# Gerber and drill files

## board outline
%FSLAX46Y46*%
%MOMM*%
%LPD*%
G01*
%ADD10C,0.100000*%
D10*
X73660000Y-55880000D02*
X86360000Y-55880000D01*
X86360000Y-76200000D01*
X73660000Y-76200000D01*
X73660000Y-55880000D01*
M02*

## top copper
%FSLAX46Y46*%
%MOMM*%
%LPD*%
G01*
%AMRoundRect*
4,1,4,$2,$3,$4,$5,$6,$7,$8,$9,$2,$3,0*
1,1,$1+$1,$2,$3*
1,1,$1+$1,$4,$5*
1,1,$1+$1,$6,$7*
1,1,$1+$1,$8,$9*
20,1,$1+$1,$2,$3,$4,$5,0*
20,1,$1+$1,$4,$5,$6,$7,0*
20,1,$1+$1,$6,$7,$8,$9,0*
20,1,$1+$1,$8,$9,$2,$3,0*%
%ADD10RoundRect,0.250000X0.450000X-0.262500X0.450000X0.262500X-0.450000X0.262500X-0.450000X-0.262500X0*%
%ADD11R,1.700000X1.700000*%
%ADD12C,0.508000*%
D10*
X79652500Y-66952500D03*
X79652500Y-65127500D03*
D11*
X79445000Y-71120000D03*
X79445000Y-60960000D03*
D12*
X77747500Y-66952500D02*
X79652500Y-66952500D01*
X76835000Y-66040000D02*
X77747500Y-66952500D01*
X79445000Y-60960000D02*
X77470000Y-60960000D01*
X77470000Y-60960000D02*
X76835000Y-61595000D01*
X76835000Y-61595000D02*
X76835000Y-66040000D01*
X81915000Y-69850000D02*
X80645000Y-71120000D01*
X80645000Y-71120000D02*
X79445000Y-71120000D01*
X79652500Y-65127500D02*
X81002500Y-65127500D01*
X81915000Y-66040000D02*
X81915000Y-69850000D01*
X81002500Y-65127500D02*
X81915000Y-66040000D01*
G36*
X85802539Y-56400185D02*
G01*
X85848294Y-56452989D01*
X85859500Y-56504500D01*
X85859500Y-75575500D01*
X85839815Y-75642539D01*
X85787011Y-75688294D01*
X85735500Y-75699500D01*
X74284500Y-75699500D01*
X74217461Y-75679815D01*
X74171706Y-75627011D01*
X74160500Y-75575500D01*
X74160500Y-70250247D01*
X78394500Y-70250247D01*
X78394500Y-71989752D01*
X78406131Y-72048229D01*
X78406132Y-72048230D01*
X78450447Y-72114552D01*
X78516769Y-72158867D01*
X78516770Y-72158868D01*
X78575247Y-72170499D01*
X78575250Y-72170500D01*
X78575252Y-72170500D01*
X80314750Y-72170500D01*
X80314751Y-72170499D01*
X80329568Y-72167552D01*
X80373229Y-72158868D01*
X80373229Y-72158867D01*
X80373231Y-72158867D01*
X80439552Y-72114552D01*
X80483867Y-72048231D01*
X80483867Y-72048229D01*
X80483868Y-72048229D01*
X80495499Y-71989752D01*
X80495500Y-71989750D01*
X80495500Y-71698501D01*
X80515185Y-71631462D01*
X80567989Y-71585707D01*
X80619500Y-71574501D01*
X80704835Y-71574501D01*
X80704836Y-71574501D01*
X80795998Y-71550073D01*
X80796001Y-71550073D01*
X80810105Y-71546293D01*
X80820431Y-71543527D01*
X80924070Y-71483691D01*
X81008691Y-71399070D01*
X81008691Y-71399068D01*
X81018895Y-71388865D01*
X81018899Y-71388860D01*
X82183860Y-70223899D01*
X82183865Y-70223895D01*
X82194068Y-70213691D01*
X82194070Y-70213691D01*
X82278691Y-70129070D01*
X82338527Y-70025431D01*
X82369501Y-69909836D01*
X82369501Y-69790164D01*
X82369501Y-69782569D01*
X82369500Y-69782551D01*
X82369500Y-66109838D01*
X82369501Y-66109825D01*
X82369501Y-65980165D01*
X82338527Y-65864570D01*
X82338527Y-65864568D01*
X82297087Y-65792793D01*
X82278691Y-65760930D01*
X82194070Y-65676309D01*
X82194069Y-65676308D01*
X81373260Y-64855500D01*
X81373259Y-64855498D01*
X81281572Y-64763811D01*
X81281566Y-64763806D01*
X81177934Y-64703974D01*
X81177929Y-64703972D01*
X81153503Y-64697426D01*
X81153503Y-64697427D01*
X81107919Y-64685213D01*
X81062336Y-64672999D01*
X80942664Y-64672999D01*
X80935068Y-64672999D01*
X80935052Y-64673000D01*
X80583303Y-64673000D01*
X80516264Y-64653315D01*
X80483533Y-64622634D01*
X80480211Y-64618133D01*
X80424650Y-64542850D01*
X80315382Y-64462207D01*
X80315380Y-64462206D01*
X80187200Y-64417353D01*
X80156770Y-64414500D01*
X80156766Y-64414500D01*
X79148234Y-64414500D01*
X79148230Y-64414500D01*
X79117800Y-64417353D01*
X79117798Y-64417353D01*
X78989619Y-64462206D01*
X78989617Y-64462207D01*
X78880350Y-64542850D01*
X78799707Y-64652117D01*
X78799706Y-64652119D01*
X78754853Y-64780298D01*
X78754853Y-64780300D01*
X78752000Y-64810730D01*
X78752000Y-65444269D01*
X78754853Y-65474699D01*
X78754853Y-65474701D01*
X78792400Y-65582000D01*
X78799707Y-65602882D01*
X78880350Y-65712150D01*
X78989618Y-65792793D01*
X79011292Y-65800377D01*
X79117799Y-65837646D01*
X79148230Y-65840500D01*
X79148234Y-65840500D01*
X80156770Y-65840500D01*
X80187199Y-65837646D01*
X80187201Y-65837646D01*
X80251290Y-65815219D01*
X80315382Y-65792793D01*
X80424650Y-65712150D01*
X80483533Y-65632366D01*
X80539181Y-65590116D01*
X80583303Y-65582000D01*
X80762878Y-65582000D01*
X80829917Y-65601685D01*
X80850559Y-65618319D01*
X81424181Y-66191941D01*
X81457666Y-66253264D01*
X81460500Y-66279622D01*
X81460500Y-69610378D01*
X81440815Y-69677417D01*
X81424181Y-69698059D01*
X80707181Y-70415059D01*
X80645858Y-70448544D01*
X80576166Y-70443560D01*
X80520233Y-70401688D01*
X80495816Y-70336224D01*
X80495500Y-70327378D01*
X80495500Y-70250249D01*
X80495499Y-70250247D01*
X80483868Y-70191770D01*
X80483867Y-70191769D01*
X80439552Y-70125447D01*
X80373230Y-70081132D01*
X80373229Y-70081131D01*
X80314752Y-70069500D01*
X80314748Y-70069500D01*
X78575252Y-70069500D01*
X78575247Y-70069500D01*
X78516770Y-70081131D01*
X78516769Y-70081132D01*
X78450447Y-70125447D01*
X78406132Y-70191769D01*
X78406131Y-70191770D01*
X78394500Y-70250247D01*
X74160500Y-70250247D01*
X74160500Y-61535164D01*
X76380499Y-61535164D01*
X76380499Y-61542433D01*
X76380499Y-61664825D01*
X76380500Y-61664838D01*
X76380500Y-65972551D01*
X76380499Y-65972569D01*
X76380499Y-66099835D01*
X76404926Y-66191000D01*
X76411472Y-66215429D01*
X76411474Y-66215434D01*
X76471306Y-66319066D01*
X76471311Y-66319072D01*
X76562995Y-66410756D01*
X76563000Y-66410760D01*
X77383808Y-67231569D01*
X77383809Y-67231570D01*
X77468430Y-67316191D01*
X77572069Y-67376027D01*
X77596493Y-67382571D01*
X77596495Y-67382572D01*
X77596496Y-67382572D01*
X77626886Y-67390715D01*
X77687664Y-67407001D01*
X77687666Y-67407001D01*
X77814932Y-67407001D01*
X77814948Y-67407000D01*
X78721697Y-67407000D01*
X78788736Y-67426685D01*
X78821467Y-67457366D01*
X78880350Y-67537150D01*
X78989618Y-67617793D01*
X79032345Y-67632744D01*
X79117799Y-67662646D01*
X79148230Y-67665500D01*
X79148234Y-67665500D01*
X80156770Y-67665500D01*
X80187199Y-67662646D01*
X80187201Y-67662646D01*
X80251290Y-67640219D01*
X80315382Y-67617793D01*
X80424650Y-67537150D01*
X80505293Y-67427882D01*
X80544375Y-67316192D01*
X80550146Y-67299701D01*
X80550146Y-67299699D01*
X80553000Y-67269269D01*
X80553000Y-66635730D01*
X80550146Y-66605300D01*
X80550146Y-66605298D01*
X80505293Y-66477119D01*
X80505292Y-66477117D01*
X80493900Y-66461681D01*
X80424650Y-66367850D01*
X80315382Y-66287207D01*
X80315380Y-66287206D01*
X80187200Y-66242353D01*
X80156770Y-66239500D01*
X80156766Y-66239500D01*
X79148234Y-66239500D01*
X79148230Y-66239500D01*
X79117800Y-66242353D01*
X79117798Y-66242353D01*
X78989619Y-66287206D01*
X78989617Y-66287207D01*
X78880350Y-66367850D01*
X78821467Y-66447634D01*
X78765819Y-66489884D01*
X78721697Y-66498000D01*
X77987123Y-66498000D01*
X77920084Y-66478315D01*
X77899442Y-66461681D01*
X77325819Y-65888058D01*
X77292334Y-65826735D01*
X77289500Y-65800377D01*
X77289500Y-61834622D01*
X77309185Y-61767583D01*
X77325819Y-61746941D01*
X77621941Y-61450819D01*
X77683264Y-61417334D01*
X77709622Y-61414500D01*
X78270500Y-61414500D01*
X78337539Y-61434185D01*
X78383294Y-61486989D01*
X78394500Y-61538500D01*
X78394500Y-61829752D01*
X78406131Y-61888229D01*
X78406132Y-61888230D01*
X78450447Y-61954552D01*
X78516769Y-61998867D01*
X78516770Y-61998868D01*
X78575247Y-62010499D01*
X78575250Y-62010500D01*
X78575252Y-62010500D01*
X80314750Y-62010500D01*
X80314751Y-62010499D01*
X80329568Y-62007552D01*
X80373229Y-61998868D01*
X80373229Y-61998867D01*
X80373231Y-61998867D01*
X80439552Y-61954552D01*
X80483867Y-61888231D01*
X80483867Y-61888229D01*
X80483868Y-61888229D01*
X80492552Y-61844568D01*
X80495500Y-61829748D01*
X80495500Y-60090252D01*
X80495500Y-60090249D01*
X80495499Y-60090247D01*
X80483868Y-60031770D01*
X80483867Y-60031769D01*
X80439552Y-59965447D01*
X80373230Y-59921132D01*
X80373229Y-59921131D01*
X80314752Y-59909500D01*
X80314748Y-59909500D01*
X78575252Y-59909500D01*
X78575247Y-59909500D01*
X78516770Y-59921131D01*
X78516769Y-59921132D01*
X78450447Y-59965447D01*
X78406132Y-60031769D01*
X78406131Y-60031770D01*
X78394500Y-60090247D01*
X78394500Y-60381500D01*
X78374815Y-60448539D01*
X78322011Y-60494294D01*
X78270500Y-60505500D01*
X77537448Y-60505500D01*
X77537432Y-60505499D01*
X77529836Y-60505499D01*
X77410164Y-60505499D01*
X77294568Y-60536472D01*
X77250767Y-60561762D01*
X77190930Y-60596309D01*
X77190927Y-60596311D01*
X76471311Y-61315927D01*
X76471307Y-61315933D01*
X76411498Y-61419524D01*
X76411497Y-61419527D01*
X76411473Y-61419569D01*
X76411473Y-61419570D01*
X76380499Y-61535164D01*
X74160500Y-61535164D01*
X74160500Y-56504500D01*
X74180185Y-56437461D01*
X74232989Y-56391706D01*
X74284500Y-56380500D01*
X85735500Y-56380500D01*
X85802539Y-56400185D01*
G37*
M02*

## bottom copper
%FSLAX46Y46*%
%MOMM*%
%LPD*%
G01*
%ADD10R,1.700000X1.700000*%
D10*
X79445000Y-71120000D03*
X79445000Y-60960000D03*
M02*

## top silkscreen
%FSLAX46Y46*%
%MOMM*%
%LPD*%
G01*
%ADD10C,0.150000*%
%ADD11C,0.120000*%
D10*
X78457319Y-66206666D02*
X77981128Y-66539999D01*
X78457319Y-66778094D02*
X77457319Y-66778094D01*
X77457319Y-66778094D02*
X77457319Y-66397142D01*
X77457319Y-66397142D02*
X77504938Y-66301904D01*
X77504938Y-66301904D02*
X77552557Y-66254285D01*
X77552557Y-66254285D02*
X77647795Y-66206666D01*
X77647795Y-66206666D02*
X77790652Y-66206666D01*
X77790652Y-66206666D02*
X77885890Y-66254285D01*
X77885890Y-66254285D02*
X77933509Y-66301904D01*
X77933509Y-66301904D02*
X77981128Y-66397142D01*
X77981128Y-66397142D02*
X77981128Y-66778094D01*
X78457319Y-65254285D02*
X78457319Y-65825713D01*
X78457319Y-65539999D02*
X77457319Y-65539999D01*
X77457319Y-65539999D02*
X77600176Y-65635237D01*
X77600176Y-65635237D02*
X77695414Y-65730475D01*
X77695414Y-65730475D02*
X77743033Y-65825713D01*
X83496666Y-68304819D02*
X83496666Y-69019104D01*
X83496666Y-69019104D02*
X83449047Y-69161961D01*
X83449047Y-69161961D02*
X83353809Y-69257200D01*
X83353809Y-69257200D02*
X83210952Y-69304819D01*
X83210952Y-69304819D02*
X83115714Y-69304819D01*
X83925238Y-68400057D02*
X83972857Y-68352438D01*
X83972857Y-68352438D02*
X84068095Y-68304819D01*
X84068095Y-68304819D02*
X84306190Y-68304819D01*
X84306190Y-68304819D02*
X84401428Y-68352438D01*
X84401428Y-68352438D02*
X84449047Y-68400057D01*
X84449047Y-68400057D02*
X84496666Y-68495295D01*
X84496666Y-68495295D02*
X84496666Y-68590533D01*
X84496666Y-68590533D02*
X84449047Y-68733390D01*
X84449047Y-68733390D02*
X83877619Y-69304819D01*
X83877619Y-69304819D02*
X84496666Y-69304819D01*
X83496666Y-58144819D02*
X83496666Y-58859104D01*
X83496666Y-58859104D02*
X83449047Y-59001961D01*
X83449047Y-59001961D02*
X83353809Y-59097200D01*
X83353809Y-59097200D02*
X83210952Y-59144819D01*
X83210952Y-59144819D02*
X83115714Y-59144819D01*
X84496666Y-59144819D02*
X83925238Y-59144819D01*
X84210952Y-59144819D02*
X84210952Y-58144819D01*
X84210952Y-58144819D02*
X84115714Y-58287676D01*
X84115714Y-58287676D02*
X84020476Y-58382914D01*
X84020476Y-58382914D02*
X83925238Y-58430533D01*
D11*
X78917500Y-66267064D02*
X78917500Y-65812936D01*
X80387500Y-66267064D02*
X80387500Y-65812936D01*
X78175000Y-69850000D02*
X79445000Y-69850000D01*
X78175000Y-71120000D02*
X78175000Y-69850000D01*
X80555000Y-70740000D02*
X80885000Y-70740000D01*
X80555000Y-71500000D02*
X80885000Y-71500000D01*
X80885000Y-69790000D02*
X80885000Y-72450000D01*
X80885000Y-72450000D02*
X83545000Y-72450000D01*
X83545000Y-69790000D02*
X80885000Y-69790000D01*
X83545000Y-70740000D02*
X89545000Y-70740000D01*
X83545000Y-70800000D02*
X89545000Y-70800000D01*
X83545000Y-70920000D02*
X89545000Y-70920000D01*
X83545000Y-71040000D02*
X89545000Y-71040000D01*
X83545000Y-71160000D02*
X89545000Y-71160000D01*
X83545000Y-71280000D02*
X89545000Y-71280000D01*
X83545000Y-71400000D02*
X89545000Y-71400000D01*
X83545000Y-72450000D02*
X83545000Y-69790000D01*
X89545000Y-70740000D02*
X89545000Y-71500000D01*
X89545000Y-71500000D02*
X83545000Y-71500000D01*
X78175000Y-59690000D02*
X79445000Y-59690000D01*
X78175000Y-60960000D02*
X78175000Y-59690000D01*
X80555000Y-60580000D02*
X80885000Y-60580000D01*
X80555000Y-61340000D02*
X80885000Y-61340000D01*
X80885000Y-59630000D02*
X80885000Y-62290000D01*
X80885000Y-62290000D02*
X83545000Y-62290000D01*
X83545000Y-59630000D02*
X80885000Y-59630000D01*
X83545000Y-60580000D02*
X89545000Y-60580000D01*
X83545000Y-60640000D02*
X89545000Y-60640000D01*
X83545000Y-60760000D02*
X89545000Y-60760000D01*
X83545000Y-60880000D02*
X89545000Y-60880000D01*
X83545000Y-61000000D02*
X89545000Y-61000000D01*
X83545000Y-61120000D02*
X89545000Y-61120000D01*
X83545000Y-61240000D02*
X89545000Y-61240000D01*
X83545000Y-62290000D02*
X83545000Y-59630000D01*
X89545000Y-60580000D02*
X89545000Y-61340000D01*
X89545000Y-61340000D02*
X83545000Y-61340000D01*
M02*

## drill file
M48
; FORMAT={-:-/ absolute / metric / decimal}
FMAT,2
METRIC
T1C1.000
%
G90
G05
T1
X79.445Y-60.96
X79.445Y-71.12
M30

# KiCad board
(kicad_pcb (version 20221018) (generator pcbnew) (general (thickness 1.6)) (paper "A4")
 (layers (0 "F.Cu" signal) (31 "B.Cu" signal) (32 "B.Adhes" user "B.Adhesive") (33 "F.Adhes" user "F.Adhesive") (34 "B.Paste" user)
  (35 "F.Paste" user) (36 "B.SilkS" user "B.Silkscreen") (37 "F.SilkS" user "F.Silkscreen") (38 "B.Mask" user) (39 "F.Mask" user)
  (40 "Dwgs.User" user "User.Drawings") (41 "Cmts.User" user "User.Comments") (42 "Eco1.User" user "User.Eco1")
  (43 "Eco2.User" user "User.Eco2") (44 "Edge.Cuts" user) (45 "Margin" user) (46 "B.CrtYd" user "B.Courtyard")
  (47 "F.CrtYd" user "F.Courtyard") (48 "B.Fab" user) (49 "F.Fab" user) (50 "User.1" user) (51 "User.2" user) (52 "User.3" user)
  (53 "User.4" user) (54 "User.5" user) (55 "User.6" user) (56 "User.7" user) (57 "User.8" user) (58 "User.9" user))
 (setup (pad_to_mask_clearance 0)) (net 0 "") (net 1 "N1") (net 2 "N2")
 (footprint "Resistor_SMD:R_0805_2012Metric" (layer "F.Cu") (at 79.6525 66.04 90)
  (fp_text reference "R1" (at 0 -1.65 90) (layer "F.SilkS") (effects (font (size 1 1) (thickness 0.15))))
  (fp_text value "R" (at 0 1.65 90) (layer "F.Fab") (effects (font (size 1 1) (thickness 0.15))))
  (fp_line (start -0.227064 -0.735) (end 0.227064 -0.735) (stroke (width 0.12) (type solid)) (layer "F.SilkS"))
  (fp_line (start -0.227064 0.735) (end 0.227064 0.735) (stroke (width 0.12) (type solid)) (layer "F.SilkS"))
  (pad "1" smd roundrect (at -0.9125 0 90) (size 1.025 1.4) (layers "F.Cu" "F.Paste" "F.Mask") (roundrect_rratio 0.243902) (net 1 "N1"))
  (pad "2" smd roundrect (at 0.9125 0 90) (size 1.025 1.4) (layers "F.Cu" "F.Paste" "F.Mask") (roundrect_rratio 0.243902) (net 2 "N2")))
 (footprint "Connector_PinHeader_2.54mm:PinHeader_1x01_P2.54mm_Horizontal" (layer "F.Cu") (at 79.445 71.12)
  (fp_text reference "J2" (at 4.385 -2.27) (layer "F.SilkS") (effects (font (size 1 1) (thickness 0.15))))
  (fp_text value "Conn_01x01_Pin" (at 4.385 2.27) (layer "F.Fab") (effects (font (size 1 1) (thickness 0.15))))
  (fp_line (start -1.27 -1.27) (end 0 -1.27) (stroke (width 0.12) (type solid)) (layer "F.SilkS"))
  (fp_line (start -1.27 0) (end -1.27 -1.27) (stroke (width 0.12) (type solid)) (layer "F.SilkS"))
  (fp_line (start 1.11 -0.38) (end 1.44 -0.38) (stroke (width 0.12) (type solid)) (layer "F.SilkS"))
  (fp_line (start 1.11 0.38) (end 1.44 0.38) (stroke (width 0.12) (type solid)) (layer "F.SilkS"))
  (fp_line (start 1.44 -1.33) (end 1.44 1.33) (stroke (width 0.12) (type solid)) (layer "F.SilkS"))
  (fp_line (start 1.44 1.33) (end 4.1 1.33) (stroke (width 0.12) (type solid)) (layer "F.SilkS"))
  (fp_line (start 4.1 -1.33) (end 1.44 -1.33) (stroke (width 0.12) (type solid)) (layer "F.SilkS"))
  (fp_line (start 4.1 -0.38) (end 10.1 -0.38) (stroke (width 0.12) (type solid)) (layer "F.SilkS"))
  (fp_line (start 4.1 -0.32) (end 10.1 -0.32) (stroke (width 0.12) (type solid)) (layer "F.SilkS"))
  (fp_line (start 4.1 -0.2) (end 10.1 -0.2) (stroke (width 0.12) (type solid)) (layer "F.SilkS"))
  (fp_line (start 4.1 -0.08) (end 10.1 -0.08) (stroke (width 0.12) (type solid)) (layer "F.SilkS"))
  (fp_line (start 4.1 0.04) (end 10.1 0.04) (stroke (width 0.12) (type solid)) (layer "F.SilkS"))
  (fp_line (start 4.1 0.16) (end 10.1 0.16) (stroke (width 0.12) (type solid)) (layer "F.SilkS"))
  (fp_line (start 4.1 0.28) (end 10.1 0.28) (stroke (width 0.12) (type solid)) (layer "F.SilkS"))
  (fp_line (start 4.1 1.33) (end 4.1 -1.33) (stroke (width 0.12) (type solid)) (layer "F.SilkS"))
  (fp_line (start 10.1 -0.38) (end 10.1 0.38) (stroke (width 0.12) (type solid)) (layer "F.SilkS"))
  (fp_line (start 10.1 0.38) (end 4.1 0.38) (stroke (width 0.12) (type solid)) (layer "F.SilkS"))
  (pad "1" thru_hole rect (at 0 0) (size 1.7 1.7) (drill 1) (layers "*.Cu" "*.Mask") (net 2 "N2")))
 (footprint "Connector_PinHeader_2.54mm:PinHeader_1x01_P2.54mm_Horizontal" (layer "F.Cu") (at 79.445 60.96)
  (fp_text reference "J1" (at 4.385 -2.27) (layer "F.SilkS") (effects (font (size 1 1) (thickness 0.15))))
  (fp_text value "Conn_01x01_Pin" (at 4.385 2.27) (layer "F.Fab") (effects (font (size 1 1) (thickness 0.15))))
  (fp_line (start -1.27 -1.27) (end 0 -1.27) (stroke (width 0.12) (type solid)) (layer "F.SilkS"))
  (fp_line (start -1.27 0) (end -1.27 -1.27) (stroke (width 0.12) (type solid)) (layer "F.SilkS"))
  (fp_line (start 1.11 -0.38) (end 1.44 -0.38) (stroke (width 0.12) (type solid)) (layer "F.SilkS"))
  (fp_line (start 1.11 0.38) (end 1.44 0.38) (stroke (width 0.12) (type solid)) (layer "F.SilkS"))
  (fp_line (start 1.44 -1.33) (end 1.44 1.33) (stroke (width 0.12) (type solid)) (layer "F.SilkS"))
  (fp_line (start 1.44 1.33) (end 4.1 1.33) (stroke (width 0.12) (type solid)) (layer "F.SilkS"))
  (fp_line (start 4.1 -1.33) (end 1.44 -1.33) (stroke (width 0.12) (type solid)) (layer "F.SilkS"))
  (fp_line (start 4.1 -0.38) (end 10.1 -0.38) (stroke (width 0.12) (type solid)) (layer "F.SilkS"))
  (fp_line (start 4.1 -0.32) (end 10.1 -0.32) (stroke (width 0.12) (type solid)) (layer "F.SilkS"))
  (fp_line (start 4.1 -0.2) (end 10.1 -0.2) (stroke (width 0.12) (type solid)) (layer "F.SilkS"))
  (fp_line (start 4.1 -0.08) (end 10.1 -0.08) (stroke (width 0.12) (type solid)) (layer "F.SilkS"))
  (fp_line (start 4.1 0.04) (end 10.1 0.04) (stroke (width 0.12) (type solid)) (layer "F.SilkS"))
  (fp_line (start 4.1 0.16) (end 10.1 0.16) (stroke (width 0.12) (type solid)) (layer "F.SilkS"))
  (fp_line (start 4.1 0.28) (end 10.1 0.28) (stroke (width 0.12) (type solid)) (layer "F.SilkS"))
  (fp_line (start 4.1 1.33) (end 4.1 -1.33) (stroke (width 0.12) (type solid)) (layer "F.SilkS"))
  (fp_line (start 10.1 -0.38) (end 10.1 0.38) (stroke (width 0.12) (type solid)) (layer "F.SilkS"))
  (fp_line (start 10.1 0.38) (end 4.1 0.38) (stroke (width 0.12) (type solid)) (layer "F.SilkS"))
  (pad "1" thru_hole rect (at 0 0) (size 1.7 1.7) (drill 1) (layers "*.Cu" "*.Mask") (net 1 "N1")))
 (gr_rect (start 73.66 55.88) (end 86.36 76.2) (stroke (width 0.1) (type default)) (fill none) (layer "Edge.Cuts"))
 (segment (start 77.7475 66.9525) (end 79.6525 66.9525) (width 0.508) (layer "F.Cu") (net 1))
 (segment (start 76.835 66.04) (end 77.7475 66.9525) (width 0.508) (layer "F.Cu") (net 1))
 (segment (start 79.445 60.96) (end 77.47 60.96) (width 0.508) (layer "F.Cu") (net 1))
 (segment (start 77.47 60.96) (end 76.835 61.595) (width 0.508) (layer "F.Cu") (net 1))
 (segment (start 76.835 61.595) (end 76.835 66.04) (width 0.508) (layer "F.Cu") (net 1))
 (segment (start 81.915 69.85) (end 80.645 71.12) (width 0.508) (layer "F.Cu") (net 2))
 (segment (start 80.645 71.12) (end 79.445 71.12) (width 0.508) (layer "F.Cu") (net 2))
 (segment (start 79.6525 65.1275) (end 81.0025 65.1275) (width 0.508) (layer "F.Cu") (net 2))
 (segment (start 81.915 66.04) (end 81.915 69.85) (width 0.508) (layer "F.Cu") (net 2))
 (segment (start 81.0025 65.1275) (end 81.915 66.04) (width 0.508) (layer "F.Cu") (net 2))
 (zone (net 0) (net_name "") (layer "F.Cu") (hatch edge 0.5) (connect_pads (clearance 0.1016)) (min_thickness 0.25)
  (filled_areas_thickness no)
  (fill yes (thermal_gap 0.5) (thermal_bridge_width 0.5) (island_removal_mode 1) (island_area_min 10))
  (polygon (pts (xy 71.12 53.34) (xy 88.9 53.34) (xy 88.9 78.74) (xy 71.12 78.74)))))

